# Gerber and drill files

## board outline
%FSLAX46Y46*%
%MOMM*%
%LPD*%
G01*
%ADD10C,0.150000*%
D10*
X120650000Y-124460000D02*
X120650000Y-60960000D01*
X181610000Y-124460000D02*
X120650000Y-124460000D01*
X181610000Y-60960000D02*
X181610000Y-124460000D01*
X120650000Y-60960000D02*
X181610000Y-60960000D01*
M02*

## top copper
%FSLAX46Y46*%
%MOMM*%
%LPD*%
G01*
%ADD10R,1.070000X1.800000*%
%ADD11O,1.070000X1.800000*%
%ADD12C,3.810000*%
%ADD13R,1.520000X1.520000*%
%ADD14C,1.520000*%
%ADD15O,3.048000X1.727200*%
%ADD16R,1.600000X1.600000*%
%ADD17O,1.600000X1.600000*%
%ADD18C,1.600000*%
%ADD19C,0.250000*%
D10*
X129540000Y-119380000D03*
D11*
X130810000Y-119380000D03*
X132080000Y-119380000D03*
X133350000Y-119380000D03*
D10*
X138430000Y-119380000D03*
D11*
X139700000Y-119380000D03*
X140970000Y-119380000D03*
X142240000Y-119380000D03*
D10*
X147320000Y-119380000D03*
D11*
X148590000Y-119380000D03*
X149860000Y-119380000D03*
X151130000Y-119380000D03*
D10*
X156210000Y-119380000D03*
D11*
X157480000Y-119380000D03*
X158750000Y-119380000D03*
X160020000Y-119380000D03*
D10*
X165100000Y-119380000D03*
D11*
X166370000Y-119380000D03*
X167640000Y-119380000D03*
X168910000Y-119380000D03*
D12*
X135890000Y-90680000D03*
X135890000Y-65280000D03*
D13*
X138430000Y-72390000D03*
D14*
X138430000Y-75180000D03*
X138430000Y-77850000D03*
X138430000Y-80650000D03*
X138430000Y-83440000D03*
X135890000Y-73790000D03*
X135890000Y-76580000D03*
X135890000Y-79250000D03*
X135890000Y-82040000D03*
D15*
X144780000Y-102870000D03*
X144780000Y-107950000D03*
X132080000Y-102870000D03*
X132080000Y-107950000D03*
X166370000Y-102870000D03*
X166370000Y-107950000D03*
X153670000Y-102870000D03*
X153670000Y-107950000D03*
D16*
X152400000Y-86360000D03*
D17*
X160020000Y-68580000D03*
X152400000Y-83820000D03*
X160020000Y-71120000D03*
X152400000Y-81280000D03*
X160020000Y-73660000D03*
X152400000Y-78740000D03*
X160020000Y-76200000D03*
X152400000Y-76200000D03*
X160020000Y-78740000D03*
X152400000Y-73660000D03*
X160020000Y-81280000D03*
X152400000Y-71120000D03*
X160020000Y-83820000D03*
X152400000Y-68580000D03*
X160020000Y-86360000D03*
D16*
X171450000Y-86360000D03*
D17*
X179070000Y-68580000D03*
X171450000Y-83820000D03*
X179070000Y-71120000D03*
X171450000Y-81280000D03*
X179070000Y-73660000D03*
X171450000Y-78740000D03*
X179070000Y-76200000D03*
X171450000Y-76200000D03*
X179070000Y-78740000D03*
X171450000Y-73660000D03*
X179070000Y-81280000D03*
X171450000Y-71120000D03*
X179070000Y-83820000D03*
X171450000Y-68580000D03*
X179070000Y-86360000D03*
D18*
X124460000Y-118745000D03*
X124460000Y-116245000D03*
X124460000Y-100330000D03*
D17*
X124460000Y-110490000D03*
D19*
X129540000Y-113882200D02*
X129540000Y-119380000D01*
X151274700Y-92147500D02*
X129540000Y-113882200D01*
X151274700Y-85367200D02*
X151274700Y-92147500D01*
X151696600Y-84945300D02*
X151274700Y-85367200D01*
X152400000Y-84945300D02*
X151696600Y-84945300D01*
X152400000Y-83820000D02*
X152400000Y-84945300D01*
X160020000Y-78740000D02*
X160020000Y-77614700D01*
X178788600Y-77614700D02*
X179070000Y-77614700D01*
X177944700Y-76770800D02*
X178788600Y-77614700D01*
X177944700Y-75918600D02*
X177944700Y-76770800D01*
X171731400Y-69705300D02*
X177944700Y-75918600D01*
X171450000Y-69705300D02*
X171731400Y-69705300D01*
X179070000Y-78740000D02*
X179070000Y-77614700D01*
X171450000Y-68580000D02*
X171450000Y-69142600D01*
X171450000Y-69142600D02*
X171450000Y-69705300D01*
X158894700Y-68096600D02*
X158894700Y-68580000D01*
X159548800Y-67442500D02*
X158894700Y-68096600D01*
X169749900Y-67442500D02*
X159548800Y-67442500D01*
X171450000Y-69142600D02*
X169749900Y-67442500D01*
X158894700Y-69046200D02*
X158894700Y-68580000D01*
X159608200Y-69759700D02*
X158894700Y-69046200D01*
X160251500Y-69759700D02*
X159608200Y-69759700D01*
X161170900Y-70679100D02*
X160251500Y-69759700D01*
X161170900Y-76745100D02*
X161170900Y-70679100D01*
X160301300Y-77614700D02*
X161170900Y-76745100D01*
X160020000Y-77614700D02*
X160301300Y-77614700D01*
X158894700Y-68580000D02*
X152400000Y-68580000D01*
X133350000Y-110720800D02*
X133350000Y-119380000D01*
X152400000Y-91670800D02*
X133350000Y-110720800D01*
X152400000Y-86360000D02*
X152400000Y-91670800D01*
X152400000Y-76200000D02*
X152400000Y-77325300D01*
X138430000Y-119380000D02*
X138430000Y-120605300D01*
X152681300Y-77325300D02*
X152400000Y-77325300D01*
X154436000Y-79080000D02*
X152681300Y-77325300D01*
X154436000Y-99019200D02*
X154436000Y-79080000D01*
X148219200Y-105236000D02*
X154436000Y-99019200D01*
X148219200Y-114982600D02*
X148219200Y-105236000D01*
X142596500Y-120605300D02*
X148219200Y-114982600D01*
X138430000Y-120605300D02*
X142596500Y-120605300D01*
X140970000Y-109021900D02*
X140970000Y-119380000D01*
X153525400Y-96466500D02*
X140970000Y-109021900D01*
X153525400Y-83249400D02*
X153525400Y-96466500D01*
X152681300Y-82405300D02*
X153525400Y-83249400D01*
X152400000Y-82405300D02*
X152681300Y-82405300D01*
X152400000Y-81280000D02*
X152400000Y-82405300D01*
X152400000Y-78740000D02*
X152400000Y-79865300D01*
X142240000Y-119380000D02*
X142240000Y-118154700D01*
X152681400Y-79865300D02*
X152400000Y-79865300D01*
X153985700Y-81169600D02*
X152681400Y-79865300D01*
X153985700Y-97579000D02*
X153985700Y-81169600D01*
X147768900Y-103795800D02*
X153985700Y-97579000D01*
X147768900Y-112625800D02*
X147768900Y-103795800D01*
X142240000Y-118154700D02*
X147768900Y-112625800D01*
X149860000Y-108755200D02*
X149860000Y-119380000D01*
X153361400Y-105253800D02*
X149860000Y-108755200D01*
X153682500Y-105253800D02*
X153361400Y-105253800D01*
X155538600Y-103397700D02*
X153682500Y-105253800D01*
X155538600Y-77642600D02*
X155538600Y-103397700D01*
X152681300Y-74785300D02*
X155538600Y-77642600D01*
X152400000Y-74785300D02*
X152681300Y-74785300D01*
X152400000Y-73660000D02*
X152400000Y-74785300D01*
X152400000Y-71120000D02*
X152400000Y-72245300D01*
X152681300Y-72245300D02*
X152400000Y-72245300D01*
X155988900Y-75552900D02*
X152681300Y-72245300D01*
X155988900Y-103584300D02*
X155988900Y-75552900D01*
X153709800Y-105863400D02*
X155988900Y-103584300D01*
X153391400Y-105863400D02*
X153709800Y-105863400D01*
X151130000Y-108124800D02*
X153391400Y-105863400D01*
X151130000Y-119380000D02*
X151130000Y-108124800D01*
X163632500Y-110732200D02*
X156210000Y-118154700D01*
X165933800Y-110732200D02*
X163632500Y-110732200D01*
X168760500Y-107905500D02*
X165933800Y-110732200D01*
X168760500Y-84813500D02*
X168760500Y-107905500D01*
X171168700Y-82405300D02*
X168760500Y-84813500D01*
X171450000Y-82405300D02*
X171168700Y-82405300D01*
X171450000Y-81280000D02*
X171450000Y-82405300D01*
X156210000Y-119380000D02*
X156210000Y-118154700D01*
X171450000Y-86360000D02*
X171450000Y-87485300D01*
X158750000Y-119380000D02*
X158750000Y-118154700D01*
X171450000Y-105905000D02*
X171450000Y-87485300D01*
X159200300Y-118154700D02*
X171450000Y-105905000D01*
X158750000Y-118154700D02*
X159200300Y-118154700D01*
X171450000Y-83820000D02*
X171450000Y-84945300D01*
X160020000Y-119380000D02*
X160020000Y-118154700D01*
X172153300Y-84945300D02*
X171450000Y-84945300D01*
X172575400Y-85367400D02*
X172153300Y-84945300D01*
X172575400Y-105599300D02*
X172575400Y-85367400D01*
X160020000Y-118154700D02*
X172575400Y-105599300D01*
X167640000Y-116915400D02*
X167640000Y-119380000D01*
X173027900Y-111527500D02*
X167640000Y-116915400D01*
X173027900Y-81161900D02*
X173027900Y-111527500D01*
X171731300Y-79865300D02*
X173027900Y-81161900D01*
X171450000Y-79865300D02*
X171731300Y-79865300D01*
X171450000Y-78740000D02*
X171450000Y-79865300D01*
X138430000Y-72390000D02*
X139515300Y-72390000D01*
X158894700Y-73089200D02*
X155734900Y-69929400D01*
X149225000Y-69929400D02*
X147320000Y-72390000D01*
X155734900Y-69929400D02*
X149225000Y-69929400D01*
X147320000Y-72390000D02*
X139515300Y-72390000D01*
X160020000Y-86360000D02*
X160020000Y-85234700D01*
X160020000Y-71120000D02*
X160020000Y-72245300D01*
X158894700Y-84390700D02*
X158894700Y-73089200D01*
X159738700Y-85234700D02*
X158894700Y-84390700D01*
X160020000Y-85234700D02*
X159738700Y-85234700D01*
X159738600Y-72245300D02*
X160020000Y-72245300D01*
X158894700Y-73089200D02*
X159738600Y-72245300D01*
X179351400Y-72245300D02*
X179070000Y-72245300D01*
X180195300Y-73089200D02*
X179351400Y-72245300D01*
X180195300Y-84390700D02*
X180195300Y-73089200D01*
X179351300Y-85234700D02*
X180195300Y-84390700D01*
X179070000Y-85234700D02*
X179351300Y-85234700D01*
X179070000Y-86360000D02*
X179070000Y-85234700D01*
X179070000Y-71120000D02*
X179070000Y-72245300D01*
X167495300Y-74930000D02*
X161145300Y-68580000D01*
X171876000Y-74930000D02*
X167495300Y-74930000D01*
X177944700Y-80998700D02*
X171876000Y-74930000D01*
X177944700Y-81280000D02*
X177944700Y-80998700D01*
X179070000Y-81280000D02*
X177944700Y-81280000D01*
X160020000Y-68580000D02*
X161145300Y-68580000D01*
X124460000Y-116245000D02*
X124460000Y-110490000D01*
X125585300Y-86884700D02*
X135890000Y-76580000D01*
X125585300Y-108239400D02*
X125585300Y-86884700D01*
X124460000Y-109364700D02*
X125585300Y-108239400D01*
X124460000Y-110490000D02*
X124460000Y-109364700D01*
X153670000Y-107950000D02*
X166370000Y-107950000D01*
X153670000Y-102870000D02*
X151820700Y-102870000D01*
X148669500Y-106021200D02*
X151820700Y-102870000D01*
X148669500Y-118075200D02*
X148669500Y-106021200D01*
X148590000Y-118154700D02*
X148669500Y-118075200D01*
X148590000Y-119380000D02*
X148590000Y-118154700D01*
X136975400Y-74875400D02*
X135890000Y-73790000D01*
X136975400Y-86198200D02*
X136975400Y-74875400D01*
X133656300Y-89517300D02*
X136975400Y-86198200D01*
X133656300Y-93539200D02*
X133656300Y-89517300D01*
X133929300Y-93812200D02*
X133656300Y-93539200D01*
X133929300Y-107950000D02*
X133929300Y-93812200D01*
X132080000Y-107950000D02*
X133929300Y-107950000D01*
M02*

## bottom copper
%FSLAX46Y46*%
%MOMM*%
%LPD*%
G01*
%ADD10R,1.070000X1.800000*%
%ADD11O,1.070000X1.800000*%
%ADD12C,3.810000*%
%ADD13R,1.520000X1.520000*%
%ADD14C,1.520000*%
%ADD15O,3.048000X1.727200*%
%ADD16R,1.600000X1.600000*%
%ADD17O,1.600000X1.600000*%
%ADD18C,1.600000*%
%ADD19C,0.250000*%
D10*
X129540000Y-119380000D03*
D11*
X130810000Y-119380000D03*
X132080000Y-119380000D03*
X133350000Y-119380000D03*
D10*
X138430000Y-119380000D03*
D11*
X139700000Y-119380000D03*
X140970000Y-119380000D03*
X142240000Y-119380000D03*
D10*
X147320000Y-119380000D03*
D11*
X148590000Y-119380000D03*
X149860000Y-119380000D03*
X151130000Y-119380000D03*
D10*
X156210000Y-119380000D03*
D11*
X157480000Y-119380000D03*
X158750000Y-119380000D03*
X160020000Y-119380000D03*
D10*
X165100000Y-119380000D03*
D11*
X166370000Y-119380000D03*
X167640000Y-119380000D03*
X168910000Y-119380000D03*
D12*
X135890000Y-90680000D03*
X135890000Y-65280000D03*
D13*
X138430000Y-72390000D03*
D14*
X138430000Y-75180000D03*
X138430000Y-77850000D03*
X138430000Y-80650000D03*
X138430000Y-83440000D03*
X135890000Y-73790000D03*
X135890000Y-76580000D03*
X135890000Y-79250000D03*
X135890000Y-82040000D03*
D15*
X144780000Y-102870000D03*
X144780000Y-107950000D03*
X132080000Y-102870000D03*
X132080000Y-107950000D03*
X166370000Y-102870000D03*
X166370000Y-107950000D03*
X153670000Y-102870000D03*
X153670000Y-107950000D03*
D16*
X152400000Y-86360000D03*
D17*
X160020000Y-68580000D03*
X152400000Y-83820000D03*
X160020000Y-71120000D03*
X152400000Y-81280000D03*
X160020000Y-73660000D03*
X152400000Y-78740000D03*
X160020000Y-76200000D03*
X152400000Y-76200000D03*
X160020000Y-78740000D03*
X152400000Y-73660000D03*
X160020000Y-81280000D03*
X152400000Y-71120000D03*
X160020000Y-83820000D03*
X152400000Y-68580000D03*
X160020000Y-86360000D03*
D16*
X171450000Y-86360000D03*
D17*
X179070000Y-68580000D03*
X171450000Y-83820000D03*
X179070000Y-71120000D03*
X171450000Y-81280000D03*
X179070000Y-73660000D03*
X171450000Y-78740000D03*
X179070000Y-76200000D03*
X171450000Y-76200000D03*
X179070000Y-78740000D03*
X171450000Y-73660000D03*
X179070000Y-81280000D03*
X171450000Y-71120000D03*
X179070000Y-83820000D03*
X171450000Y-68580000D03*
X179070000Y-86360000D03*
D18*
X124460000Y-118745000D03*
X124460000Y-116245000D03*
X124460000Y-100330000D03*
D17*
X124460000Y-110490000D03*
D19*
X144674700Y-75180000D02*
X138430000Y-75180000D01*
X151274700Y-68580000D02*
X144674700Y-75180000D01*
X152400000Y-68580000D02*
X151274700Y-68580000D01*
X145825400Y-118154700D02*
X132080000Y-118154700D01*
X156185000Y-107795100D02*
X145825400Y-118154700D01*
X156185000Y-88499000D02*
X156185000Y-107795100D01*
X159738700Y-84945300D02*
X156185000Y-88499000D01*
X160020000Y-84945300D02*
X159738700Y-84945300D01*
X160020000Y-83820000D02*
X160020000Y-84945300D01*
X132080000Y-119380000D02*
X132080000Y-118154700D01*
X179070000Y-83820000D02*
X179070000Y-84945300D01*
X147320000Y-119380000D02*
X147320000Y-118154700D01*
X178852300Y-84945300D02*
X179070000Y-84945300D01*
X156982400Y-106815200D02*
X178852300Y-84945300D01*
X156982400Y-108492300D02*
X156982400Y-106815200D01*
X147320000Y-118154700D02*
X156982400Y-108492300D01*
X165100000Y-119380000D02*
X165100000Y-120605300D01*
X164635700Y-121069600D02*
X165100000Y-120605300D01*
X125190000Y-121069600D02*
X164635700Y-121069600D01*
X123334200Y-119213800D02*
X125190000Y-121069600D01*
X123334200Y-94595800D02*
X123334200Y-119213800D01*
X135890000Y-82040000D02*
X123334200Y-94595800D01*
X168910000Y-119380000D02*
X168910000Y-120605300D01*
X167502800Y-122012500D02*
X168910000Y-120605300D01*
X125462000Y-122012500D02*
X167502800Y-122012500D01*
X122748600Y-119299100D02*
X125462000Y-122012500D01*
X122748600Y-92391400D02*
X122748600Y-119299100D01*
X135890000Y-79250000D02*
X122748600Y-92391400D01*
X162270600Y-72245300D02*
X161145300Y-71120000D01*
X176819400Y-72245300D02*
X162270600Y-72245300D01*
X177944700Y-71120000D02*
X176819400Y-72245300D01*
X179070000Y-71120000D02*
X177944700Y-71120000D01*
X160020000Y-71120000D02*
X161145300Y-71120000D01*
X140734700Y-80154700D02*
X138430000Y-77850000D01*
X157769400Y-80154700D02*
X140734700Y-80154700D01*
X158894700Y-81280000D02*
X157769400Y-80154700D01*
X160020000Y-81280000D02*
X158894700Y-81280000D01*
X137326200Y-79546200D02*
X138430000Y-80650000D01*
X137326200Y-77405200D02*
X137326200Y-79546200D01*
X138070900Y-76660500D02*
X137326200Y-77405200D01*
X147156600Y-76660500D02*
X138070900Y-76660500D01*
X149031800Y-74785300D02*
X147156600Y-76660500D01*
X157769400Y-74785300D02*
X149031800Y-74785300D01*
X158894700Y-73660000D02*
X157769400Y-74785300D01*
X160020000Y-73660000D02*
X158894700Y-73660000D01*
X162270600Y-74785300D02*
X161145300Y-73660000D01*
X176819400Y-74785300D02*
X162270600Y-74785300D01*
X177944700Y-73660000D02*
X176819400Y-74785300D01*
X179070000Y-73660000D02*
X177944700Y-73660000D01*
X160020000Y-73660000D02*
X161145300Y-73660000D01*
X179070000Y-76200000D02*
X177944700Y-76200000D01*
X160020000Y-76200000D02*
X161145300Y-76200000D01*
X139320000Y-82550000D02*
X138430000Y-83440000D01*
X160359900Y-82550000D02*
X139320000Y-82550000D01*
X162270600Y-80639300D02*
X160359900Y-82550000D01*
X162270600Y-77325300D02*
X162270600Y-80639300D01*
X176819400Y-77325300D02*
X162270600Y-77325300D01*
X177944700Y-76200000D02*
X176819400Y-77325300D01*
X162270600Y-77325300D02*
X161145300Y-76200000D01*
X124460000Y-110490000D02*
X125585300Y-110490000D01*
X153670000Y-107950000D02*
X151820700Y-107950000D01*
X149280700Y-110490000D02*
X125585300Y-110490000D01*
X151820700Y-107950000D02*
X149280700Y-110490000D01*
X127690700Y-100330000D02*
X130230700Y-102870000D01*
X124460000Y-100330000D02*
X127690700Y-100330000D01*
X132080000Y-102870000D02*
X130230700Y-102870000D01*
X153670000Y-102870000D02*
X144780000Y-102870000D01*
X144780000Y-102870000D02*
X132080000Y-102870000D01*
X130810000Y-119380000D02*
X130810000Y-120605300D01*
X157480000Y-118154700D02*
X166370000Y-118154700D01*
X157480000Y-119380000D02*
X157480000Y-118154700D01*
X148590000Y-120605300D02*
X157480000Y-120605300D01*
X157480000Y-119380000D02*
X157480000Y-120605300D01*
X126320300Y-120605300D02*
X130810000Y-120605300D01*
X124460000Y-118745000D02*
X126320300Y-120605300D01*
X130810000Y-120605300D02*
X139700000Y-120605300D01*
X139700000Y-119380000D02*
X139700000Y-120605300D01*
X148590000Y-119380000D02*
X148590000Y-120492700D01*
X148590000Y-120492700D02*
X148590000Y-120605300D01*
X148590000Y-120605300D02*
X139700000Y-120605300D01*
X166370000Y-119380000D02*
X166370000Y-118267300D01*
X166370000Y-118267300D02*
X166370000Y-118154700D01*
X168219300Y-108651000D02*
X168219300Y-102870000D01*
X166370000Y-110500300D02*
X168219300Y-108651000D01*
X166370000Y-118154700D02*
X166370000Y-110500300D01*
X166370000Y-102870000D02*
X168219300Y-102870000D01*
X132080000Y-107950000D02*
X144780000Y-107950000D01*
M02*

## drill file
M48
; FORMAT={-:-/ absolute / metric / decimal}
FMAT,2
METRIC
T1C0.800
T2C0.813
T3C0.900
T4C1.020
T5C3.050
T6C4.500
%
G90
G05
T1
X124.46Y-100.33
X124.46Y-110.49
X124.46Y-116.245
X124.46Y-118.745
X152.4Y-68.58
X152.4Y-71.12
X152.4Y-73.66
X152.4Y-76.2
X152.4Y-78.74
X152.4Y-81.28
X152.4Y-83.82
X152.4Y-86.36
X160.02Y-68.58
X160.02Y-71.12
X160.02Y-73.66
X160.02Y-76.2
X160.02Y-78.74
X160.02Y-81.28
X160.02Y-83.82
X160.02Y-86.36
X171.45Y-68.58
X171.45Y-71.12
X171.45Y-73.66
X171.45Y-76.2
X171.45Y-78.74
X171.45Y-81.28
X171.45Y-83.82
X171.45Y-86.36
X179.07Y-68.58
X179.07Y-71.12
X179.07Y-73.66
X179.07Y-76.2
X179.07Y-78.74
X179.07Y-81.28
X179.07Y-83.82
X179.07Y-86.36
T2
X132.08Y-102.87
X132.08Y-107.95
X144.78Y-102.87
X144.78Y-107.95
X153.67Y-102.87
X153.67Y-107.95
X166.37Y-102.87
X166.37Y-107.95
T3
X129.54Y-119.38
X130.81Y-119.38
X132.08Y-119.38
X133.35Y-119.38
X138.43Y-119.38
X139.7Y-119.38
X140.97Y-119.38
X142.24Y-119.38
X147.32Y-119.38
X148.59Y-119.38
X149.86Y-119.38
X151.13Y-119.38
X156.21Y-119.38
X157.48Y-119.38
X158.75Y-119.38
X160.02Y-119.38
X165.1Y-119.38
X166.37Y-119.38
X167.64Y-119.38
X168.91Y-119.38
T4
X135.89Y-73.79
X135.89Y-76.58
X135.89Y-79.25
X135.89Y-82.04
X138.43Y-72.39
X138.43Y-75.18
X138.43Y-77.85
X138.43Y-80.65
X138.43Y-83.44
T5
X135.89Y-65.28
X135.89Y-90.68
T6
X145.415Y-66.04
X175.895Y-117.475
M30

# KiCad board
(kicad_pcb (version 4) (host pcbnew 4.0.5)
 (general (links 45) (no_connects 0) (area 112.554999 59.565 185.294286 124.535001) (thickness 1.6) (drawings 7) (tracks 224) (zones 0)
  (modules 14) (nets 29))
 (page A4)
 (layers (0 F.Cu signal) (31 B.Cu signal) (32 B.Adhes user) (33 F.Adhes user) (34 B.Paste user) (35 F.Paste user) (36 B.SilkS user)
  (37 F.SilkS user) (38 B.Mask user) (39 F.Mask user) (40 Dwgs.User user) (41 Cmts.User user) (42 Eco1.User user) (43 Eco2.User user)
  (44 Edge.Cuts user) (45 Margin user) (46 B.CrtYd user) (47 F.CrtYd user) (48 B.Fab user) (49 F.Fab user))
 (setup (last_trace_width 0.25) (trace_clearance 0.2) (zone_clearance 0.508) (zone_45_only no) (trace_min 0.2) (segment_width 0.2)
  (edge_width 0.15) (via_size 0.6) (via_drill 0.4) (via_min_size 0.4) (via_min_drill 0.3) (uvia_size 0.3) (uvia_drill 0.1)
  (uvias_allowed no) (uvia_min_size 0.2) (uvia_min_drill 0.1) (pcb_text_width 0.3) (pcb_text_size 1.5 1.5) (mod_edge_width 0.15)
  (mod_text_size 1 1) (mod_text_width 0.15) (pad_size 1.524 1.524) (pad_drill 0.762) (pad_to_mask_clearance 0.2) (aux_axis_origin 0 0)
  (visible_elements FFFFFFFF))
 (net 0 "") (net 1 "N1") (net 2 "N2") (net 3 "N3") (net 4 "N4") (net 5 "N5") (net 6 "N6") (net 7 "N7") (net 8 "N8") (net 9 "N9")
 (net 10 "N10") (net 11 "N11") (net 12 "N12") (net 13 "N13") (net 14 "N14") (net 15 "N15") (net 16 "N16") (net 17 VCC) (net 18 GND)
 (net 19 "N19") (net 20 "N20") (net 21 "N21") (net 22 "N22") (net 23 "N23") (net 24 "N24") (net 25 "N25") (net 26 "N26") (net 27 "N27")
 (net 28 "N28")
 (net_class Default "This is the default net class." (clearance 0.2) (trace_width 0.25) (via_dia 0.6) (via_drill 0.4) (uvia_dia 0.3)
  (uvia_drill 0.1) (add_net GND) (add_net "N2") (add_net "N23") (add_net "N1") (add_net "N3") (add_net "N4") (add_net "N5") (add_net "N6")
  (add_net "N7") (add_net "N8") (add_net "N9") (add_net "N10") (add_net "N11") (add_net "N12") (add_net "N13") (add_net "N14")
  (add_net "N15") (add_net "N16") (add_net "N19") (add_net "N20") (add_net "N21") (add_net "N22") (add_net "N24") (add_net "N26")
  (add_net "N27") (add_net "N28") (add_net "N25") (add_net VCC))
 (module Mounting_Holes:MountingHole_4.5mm (layer F.Cu) (at 145.415 66.04)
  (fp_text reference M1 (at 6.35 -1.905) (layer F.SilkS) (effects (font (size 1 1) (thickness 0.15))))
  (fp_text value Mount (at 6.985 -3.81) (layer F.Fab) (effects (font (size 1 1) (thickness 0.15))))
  (pad 1 np_thru_hole circle (at 0 0) (size 4.5 4.5) (drill 4.5) (layers *.Cu *.Mask)))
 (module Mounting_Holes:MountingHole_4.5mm (layer F.Cu) (at 175.895 117.475)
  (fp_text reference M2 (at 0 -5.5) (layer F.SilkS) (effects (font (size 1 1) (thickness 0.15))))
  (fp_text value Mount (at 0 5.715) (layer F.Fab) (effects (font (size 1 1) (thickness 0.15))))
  (pad 1 np_thru_hole circle (at 0 0) (size 4.5 4.5) (drill 4.5) (layers *.Cu *.Mask)))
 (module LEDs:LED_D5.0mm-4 (layer F.Cu) (at 129.54 119.38)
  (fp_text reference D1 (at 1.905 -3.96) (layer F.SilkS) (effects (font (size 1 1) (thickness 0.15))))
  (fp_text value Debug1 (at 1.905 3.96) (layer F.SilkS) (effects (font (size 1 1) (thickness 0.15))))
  (pad 1 thru_hole rect (at 0 0) (size 1.07 1.8) (drill 0.9) (layers *.Cu *.Mask) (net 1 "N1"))
  (pad 2 thru_hole oval (at 1.27 0) (size 1.07 1.8) (drill 0.9) (layers *.Cu *.Mask) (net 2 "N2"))
  (pad 3 thru_hole oval (at 2.54 0) (size 1.07 1.8) (drill 0.9) (layers *.Cu *.Mask) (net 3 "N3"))
  (pad 4 thru_hole oval (at 3.81 0) (size 1.07 1.8) (drill 0.9) (layers *.Cu *.Mask) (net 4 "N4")))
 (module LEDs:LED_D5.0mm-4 (layer F.Cu) (at 138.43 119.38)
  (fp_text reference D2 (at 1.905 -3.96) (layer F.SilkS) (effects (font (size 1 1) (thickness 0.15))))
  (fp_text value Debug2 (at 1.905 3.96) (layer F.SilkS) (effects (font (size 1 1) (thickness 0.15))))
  (pad 1 thru_hole rect (at 0 0) (size 1.07 1.8) (drill 0.9) (layers *.Cu *.Mask) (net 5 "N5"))
  (pad 2 thru_hole oval (at 1.27 0) (size 1.07 1.8) (drill 0.9) (layers *.Cu *.Mask) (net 2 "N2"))
  (pad 3 thru_hole oval (at 2.54 0) (size 1.07 1.8) (drill 0.9) (layers *.Cu *.Mask) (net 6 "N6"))
  (pad 4 thru_hole oval (at 3.81 0) (size 1.07 1.8) (drill 0.9) (layers *.Cu *.Mask) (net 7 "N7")))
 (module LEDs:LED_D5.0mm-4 (layer F.Cu) (at 147.32 119.38)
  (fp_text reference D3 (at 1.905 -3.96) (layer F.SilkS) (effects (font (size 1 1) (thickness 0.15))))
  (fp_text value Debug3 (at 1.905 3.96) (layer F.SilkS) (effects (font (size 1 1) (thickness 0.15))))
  (pad 1 thru_hole rect (at 0 0) (size 1.07 1.8) (drill 0.9) (layers *.Cu *.Mask) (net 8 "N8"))
  (pad 2 thru_hole oval (at 1.27 0) (size 1.07 1.8) (drill 0.9) (layers *.Cu *.Mask) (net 2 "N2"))
  (pad 3 thru_hole oval (at 2.54 0) (size 1.07 1.8) (drill 0.9) (layers *.Cu *.Mask) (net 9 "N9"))
  (pad 4 thru_hole oval (at 3.81 0) (size 1.07 1.8) (drill 0.9) (layers *.Cu *.Mask) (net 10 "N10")))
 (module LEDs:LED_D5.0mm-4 (layer F.Cu) (at 156.21 119.38)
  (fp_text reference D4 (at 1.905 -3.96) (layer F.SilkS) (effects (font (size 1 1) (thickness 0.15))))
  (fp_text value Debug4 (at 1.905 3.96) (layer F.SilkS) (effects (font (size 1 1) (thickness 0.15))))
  (pad 1 thru_hole rect (at 0 0) (size 1.07 1.8) (drill 0.9) (layers *.Cu *.Mask) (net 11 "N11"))
  (pad 2 thru_hole oval (at 1.27 0) (size 1.07 1.8) (drill 0.9) (layers *.Cu *.Mask) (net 2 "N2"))
  (pad 3 thru_hole oval (at 2.54 0) (size 1.07 1.8) (drill 0.9) (layers *.Cu *.Mask) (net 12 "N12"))
  (pad 4 thru_hole oval (at 3.81 0) (size 1.07 1.8) (drill 0.9) (layers *.Cu *.Mask) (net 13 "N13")))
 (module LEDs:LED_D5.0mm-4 (layer F.Cu) (at 165.1 119.38)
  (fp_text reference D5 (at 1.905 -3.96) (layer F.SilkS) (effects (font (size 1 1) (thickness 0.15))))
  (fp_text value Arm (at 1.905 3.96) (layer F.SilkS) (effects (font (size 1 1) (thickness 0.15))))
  (pad 1 thru_hole rect (at 0 0) (size 1.07 1.8) (drill 0.9) (layers *.Cu *.Mask) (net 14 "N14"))
  (pad 2 thru_hole oval (at 1.27 0) (size 1.07 1.8) (drill 0.9) (layers *.Cu *.Mask) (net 2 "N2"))
  (pad 3 thru_hole oval (at 2.54 0) (size 1.07 1.8) (drill 0.9) (layers *.Cu *.Mask) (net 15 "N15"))
  (pad 4 thru_hole oval (at 3.81 0) (size 1.07 1.8) (drill 0.9) (layers *.Cu *.Mask) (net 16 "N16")))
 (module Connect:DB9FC (layer B.Cu) (at 138.43 72.39 270)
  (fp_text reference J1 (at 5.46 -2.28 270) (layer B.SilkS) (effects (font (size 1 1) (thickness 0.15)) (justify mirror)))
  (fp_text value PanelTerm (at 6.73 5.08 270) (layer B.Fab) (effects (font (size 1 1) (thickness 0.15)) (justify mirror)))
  (pad "" thru_hole circle (at 18.29 2.54 270) (size 3.81 3.81) (drill 3.05) (layers *.Cu *.Mask))
  (pad "" thru_hole circle (at -7.11 2.54 270) (size 3.81 3.81) (drill 3.05) (layers *.Cu *.Mask))
  (pad 1 thru_hole rect (at 0 0 270) (size 1.52 1.52) (drill 1.02) (layers *.Cu *.Mask) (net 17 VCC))
  (pad 2 thru_hole circle (at 2.79 0 270) (size 1.52 1.52) (drill 1.02) (layers *.Cu *.Mask) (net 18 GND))
  (pad 3 thru_hole circle (at 5.46 0 270) (size 1.52 1.52) (drill 1.02) (layers *.Cu *.Mask) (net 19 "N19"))
  (pad 4 thru_hole circle (at 8.26 0 270) (size 1.52 1.52) (drill 1.02) (layers *.Cu *.Mask) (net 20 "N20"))
  (pad 5 thru_hole circle (at 11.05 0 270) (size 1.52 1.52) (drill 1.02) (layers *.Cu *.Mask) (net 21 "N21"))
  (pad 6 thru_hole circle (at 1.4 2.54 270) (size 1.52 1.52) (drill 1.02) (layers *.Cu *.Mask) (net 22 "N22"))
  (pad 7 thru_hole circle (at 4.19 2.54 270) (size 1.52 1.52) (drill 1.02) (layers *.Cu *.Mask) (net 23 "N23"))
  (pad 8 thru_hole circle (at 6.86 2.54 270) (size 1.52 1.52) (drill 1.02) (layers *.Cu *.Mask) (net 16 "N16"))
  (pad 9 thru_hole circle (at 9.65 2.54 270) (size 1.52 1.52) (drill 1.02) (layers *.Cu *.Mask) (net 14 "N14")))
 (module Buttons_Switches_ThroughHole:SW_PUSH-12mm (layer F.Cu) (at 138.43 105.41)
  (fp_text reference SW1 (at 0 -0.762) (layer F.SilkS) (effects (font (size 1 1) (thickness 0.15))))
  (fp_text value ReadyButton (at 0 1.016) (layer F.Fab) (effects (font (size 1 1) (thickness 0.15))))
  (pad 1 thru_hole oval (at 6.35 -2.54) (size 3.048 1.7272) (drill 0.8128) (layers *.Cu *.Mask) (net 2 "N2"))
  (pad 2 thru_hole oval (at 6.35 2.54) (size 3.048 1.7272) (drill 0.8128) (layers *.Cu *.Mask) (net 22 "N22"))
  (pad 1 thru_hole oval (at -6.35 -2.54) (size 3.048 1.7272) (drill 0.8128) (layers *.Cu *.Mask) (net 2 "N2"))
  (pad 2 thru_hole oval (at -6.35 2.54) (size 3.048 1.7272) (drill 0.8128) (layers *.Cu *.Mask) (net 22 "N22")))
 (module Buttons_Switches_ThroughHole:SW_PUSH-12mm (layer F.Cu) (at 160.02 105.41)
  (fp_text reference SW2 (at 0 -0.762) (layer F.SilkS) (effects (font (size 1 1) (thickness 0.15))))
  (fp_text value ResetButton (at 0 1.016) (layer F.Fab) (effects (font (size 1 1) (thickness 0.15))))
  (pad 1 thru_hole oval (at 6.35 -2.54) (size 3.048 1.7272) (drill 0.8128) (layers *.Cu *.Mask) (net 2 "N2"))
  (pad 2 thru_hole oval (at 6.35 2.54) (size 3.048 1.7272) (drill 0.8128) (layers *.Cu *.Mask) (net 23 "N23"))
  (pad 1 thru_hole oval (at -6.35 -2.54) (size 3.048 1.7272) (drill 0.8128) (layers *.Cu *.Mask) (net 2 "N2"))
  (pad 2 thru_hole oval (at -6.35 2.54) (size 3.048 1.7272) (drill 0.8128) (layers *.Cu *.Mask) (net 23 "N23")))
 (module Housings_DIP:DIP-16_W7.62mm (layer B.Cu) (at 152.4 86.36)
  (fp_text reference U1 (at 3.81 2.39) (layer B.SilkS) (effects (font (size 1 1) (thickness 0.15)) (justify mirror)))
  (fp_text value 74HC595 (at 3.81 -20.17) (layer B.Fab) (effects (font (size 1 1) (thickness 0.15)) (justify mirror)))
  (pad 1 thru_hole rect (at 0 0) (size 1.6 1.6) (drill 0.8) (layers *.Cu *.Mask) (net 4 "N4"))
  (pad 9 thru_hole oval (at 7.62 -17.78) (size 1.6 1.6) (drill 0.8) (layers *.Cu *.Mask) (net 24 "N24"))
  (pad 2 thru_hole oval (at 0 -2.54) (size 1.6 1.6) (drill 0.8) (layers *.Cu *.Mask) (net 1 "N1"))
  (pad 10 thru_hole oval (at 7.62 -15.24) (size 1.6 1.6) (drill 0.8) (layers *.Cu *.Mask) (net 17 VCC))
  (pad 3 thru_hole oval (at 0 -5.08) (size 1.6 1.6) (drill 0.8) (layers *.Cu *.Mask) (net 6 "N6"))
  (pad 11 thru_hole oval (at 7.62 -12.7) (size 1.6 1.6) (drill 0.8) (layers *.Cu *.Mask) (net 20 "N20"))
  (pad 4 thru_hole oval (at 0 -7.62) (size 1.6 1.6) (drill 0.8) (layers *.Cu *.Mask) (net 7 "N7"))
  (pad 12 thru_hole oval (at 7.62 -10.16) (size 1.6 1.6) (drill 0.8) (layers *.Cu *.Mask) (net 21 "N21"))
  (pad 5 thru_hole oval (at 0 -10.16) (size 1.6 1.6) (drill 0.8) (layers *.Cu *.Mask) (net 5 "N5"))
  (pad 13 thru_hole oval (at 7.62 -7.62) (size 1.6 1.6) (drill 0.8) (layers *.Cu *.Mask) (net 18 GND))
  (pad 6 thru_hole oval (at 0 -12.7) (size 1.6 1.6) (drill 0.8) (layers *.Cu *.Mask) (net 9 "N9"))
  (pad 14 thru_hole oval (at 7.62 -5.08) (size 1.6 1.6) (drill 0.8) (layers *.Cu *.Mask) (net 19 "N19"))
  (pad 7 thru_hole oval (at 0 -15.24) (size 1.6 1.6) (drill 0.8) (layers *.Cu *.Mask) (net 10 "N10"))
  (pad 15 thru_hole oval (at 7.62 -2.54) (size 1.6 1.6) (drill 0.8) (layers *.Cu *.Mask) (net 3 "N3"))
  (pad 8 thru_hole oval (at 0 -17.78) (size 1.6 1.6) (drill 0.8) (layers *.Cu *.Mask) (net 18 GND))
  (pad 16 thru_hole oval (at 7.62 0) (size 1.6 1.6) (drill 0.8) (layers *.Cu *.Mask) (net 17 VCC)))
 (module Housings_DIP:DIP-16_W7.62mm (layer B.Cu) (at 171.45 86.36)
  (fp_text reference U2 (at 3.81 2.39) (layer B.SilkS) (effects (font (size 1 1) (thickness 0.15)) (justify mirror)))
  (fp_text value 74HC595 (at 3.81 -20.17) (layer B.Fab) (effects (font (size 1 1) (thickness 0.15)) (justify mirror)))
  (pad 1 thru_hole rect (at 0 0) (size 1.6 1.6) (drill 0.8) (layers *.Cu *.Mask) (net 12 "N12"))
  (pad 9 thru_hole oval (at 7.62 -17.78) (size 1.6 1.6) (drill 0.8) (layers *.Cu *.Mask) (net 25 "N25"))
  (pad 2 thru_hole oval (at 0 -2.54) (size 1.6 1.6) (drill 0.8) (layers *.Cu *.Mask) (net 13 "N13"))
  (pad 10 thru_hole oval (at 7.62 -15.24) (size 1.6 1.6) (drill 0.8) (layers *.Cu *.Mask) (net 17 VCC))
  (pad 3 thru_hole oval (at 0 -5.08) (size 1.6 1.6) (drill 0.8) (layers *.Cu *.Mask) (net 11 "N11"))
  (pad 11 thru_hole oval (at 7.62 -12.7) (size 1.6 1.6) (drill 0.8) (layers *.Cu *.Mask) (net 20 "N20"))
  (pad 4 thru_hole oval (at 0 -7.62) (size 1.6 1.6) (drill 0.8) (layers *.Cu *.Mask) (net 15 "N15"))
  (pad 12 thru_hole oval (at 7.62 -10.16) (size 1.6 1.6) (drill 0.8) (layers *.Cu *.Mask) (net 21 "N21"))
  (pad 5 thru_hole oval (at 0 -10.16) (size 1.6 1.6) (drill 0.8) (layers *.Cu *.Mask) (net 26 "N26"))
  (pad 13 thru_hole oval (at 7.62 -7.62) (size 1.6 1.6) (drill 0.8) (layers *.Cu *.Mask) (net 18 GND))
  (pad 6 thru_hole oval (at 0 -12.7) (size 1.6 1.6) (drill 0.8) (layers *.Cu *.Mask) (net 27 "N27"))
  (pad 14 thru_hole oval (at 7.62 -5.08) (size 1.6 1.6) (drill 0.8) (layers *.Cu *.Mask) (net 24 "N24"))
  (pad 7 thru_hole oval (at 0 -15.24) (size 1.6 1.6) (drill 0.8) (layers *.Cu *.Mask) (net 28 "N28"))
  (pad 15 thru_hole oval (at 7.62 -2.54) (size 1.6 1.6) (drill 0.8) (layers *.Cu *.Mask) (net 8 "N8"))
  (pad 8 thru_hole oval (at 0 -17.78) (size 1.6 1.6) (drill 0.8) (layers *.Cu *.Mask) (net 18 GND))
  (pad 16 thru_hole oval (at 7.62 0) (size 1.6 1.6) (drill 0.8) (layers *.Cu *.Mask) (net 17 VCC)))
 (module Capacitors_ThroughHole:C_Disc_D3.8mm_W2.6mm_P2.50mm (layer F.Cu) (at 124.46 118.745 90)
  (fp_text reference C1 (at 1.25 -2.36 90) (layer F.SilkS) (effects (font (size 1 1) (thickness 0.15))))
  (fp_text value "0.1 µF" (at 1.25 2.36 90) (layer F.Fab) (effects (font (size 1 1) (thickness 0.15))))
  (pad 1 thru_hole circle (at 0 0 90) (size 1.6 1.6) (drill 0.8) (layers *.Cu *.Mask) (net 2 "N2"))
  (pad 2 thru_hole circle (at 2.5 0 90) (size 1.6 1.6) (drill 0.8) (layers *.Cu *.Mask) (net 23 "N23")))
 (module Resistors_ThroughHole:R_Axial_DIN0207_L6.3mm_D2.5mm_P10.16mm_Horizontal (layer F.Cu) (at 124.46 100.33 270)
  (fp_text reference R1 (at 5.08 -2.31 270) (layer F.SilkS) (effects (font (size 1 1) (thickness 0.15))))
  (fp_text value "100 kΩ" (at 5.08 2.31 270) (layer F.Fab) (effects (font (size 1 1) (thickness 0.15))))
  (pad 1 thru_hole circle (at 0 0 270) (size 1.6 1.6) (drill 0.8) (layers *.Cu *.Mask) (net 2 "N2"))
  (pad 2 thru_hole oval (at 10.16 0 270) (size 1.6 1.6) (drill 0.8) (layers *.Cu *.Mask) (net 23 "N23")))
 (gr_line (start 120.65 124.46) (end 120.65 60.96) (angle 90) (layer Edge.Cuts) (width 0.15))
 (gr_line (start 181.61 124.46) (end 120.65 124.46) (angle 90) (layer Edge.Cuts) (width 0.15))
 (gr_line (start 181.61 60.96) (end 181.61 124.46) (angle 90) (layer Edge.Cuts) (width 0.15))
 (gr_line (start 120.65 60.96) (end 181.61 60.96) (angle 90) (layer Edge.Cuts) (width 0.15))
 (segment (start 129.54 113.8822) (end 129.54 119.38) (width 0.25) (layer F.Cu) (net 1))
 (segment (start 151.2747 92.1475) (end 129.54 113.8822) (width 0.25) (layer F.Cu) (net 1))
 (segment (start 151.2747 85.3672) (end 151.2747 92.1475) (width 0.25) (layer F.Cu) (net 1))
 (segment (start 151.6966 84.9453) (end 151.2747 85.3672) (width 0.25) (layer F.Cu) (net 1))
 (segment (start 152.4 84.9453) (end 151.6966 84.9453) (width 0.25) (layer F.Cu) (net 1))
 (segment (start 152.4 83.82) (end 152.4 84.9453) (width 0.25) (layer F.Cu) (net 1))
 (segment (start 144.6747 75.18) (end 138.43 75.18) (width 0.25) (layer B.Cu) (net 18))
 (segment (start 151.2747 68.58) (end 144.6747 75.18) (width 0.25) (layer B.Cu) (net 18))
 (segment (start 152.4 68.58) (end 151.2747 68.58) (width 0.25) (layer B.Cu) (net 18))
 (segment (start 160.02 78.74) (end 160.02 77.6147) (width 0.25) (layer F.Cu) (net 18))
 (segment (start 178.7886 77.6147) (end 179.07 77.6147) (width 0.25) (layer F.Cu) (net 18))
 (segment (start 177.9447 76.7708) (end 178.7886 77.6147) (width 0.25) (layer F.Cu) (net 18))
 (segment (start 177.9447 75.9186) (end 177.9447 76.7708) (width 0.25) (layer F.Cu) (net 18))
 (segment (start 171.7314 69.7053) (end 177.9447 75.9186) (width 0.25) (layer F.Cu) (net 18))
 (segment (start 171.45 69.7053) (end 171.7314 69.7053) (width 0.25) (layer F.Cu) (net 18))
 (segment (start 179.07 78.74) (end 179.07 77.6147) (width 0.25) (layer F.Cu) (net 18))
 (segment (start 171.45 68.58) (end 171.45 69.1426) (width 0.25) (layer F.Cu) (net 18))
 (segment (start 171.45 69.1426) (end 171.45 69.7053) (width 0.25) (layer F.Cu) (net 18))
 (segment (start 158.8947 68.0966) (end 158.8947 68.58) (width 0.25) (layer F.Cu) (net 18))
 (segment (start 159.5488 67.4425) (end 158.8947 68.0966) (width 0.25) (layer F.Cu) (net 18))
 (segment (start 169.7499 67.4425) (end 159.5488 67.4425) (width 0.25) (layer F.Cu) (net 18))
 (segment (start 171.45 69.1426) (end 169.7499 67.4425) (width 0.25) (layer F.Cu) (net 18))
 (segment (start 158.8947 69.0462) (end 158.8947 68.58) (width 0.25) (layer F.Cu) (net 18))
 (segment (start 159.6082 69.7597) (end 158.8947 69.0462) (width 0.25) (layer F.Cu) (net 18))
 (segment (start 160.2515 69.7597) (end 159.6082 69.7597) (width 0.25) (layer F.Cu) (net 18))
 (segment (start 161.1709 70.6791) (end 160.2515 69.7597) (width 0.25) (layer F.Cu) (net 18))
 (segment (start 161.1709 76.7451) (end 161.1709 70.6791) (width 0.25) (layer F.Cu) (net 18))
 (segment (start 160.3013 77.6147) (end 161.1709 76.7451) (width 0.25) (layer F.Cu) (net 18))
 (segment (start 160.02 77.6147) (end 160.3013 77.6147) (width 0.25) (layer F.Cu) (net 18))
 (segment (start 158.8947 68.58) (end 152.4 68.58) (width 0.25) (layer F.Cu) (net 18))
 (segment (start 145.8254 118.1547) (end 132.08 118.1547) (width 0.25) (layer B.Cu) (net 3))
 (segment (start 156.185 107.7951) (end 145.8254 118.1547) (width 0.25) (layer B.Cu) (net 3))
 (segment (start 156.185 88.499) (end 156.185 107.7951) (width 0.25) (layer B.Cu) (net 3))
 (segment (start 159.7387 84.9453) (end 156.185 88.499) (width 0.25) (layer B.Cu) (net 3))
 (segment (start 160.02 84.9453) (end 159.7387 84.9453) (width 0.25) (layer B.Cu) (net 3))
 (segment (start 160.02 83.82) (end 160.02 84.9453) (width 0.25) (layer B.Cu) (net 3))
 (segment (start 132.08 119.38) (end 132.08 118.1547) (width 0.25) (layer B.Cu) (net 3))
 (segment (start 133.35 110.7208) (end 133.35 119.38) (width 0.25) (layer F.Cu) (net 4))
 (segment (start 152.4 91.6708) (end 133.35 110.7208) (width 0.25) (layer F.Cu) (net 4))
 (segment (start 152.4 86.36) (end 152.4 91.6708) (width 0.25) (layer F.Cu) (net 4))
 (segment (start 152.4 76.2) (end 152.4 77.3253) (width 0.25) (layer F.Cu) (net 5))
 (segment (start 138.43 119.38) (end 138.43 120.6053) (width 0.25) (layer F.Cu) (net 5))
 (segment (start 152.6813 77.3253) (end 152.4 77.3253) (width 0.25) (layer F.Cu) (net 5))
 (segment (start 154.436 79.08) (end 152.6813 77.3253) (width 0.25) (layer F.Cu) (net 5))
 (segment (start 154.436 99.0192) (end 154.436 79.08) (width 0.25) (layer F.Cu) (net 5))
 (segment (start 148.2192 105.236) (end 154.436 99.0192) (width 0.25) (layer F.Cu) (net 5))
 (segment (start 148.2192 114.9826) (end 148.2192 105.236) (width 0.25) (layer F.Cu) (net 5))
 (segment (start 142.5965 120.6053) (end 148.2192 114.9826) (width 0.25) (layer F.Cu) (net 5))
 (segment (start 138.43 120.6053) (end 142.5965 120.6053) (width 0.25) (layer F.Cu) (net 5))
 (segment (start 140.97 109.0219) (end 140.97 119.38) (width 0.25) (layer F.Cu) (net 6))
 (segment (start 153.5254 96.4665) (end 140.97 109.0219) (width 0.25) (layer F.Cu) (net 6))
 (segment (start 153.5254 83.2494) (end 153.5254 96.4665) (width 0.25) (layer F.Cu) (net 6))
 (segment (start 152.6813 82.4053) (end 153.5254 83.2494) (width 0.25) (layer F.Cu) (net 6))
 (segment (start 152.4 82.4053) (end 152.6813 82.4053) (width 0.25) (layer F.Cu) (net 6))
 (segment (start 152.4 81.28) (end 152.4 82.4053) (width 0.25) (layer F.Cu) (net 6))
 (segment (start 152.4 78.74) (end 152.4 79.8653) (width 0.25) (layer F.Cu) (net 7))
 (segment (start 142.24 119.38) (end 142.24 118.1547) (width 0.25) (layer F.Cu) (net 7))
 (segment (start 152.6814 79.8653) (end 152.4 79.8653) (width 0.25) (layer F.Cu) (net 7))
 (segment (start 153.9857 81.1696) (end 152.6814 79.8653) (width 0.25) (layer F.Cu) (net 7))
 (segment (start 153.9857 97.579) (end 153.9857 81.1696) (width 0.25) (layer F.Cu) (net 7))
 (segment (start 147.7689 103.7958) (end 153.9857 97.579) (width 0.25) (layer F.Cu) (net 7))
 (segment (start 147.7689 112.6258) (end 147.7689 103.7958) (width 0.25) (layer F.Cu) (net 7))
 (segment (start 142.24 118.1547) (end 147.7689 112.6258) (width 0.25) (layer F.Cu) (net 7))
 (segment (start 179.07 83.82) (end 179.07 84.9453) (width 0.25) (layer B.Cu) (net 8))
 (segment (start 147.32 119.38) (end 147.32 118.1547) (width 0.25) (layer B.Cu) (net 8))
 (segment (start 178.8523 84.9453) (end 179.07 84.9453) (width 0.25) (layer B.Cu) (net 8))
 (segment (start 156.9824 106.8152) (end 178.8523 84.9453) (width 0.25) (layer B.Cu) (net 8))
 (segment (start 156.9824 108.4923) (end 156.9824 106.8152) (width 0.25) (layer B.Cu) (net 8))
 (segment (start 147.32 118.1547) (end 156.9824 108.4923) (width 0.25) (layer B.Cu) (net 8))
 (segment (start 149.86 108.7552) (end 149.86 119.38) (width 0.25) (layer F.Cu) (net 9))
 (segment (start 153.3614 105.2538) (end 149.86 108.7552) (width 0.25) (layer F.Cu) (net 9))
 (segment (start 153.6825 105.2538) (end 153.3614 105.2538) (width 0.25) (layer F.Cu) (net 9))
 (segment (start 155.5386 103.3977) (end 153.6825 105.2538) (width 0.25) (layer F.Cu) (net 9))
 (segment (start 155.5386 77.6426) (end 155.5386 103.3977) (width 0.25) (layer F.Cu) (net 9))
 (segment (start 152.6813 74.7853) (end 155.5386 77.6426) (width 0.25) (layer F.Cu) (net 9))
 (segment (start 152.4 74.7853) (end 152.6813 74.7853) (width 0.25) (layer F.Cu) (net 9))
 (segment (start 152.4 73.66) (end 152.4 74.7853) (width 0.25) (layer F.Cu) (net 9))
 (segment (start 152.4 71.12) (end 152.4 72.2453) (width 0.25) (layer F.Cu) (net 10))
 (segment (start 152.6813 72.2453) (end 152.4 72.2453) (width 0.25) (layer F.Cu) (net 10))
 (segment (start 155.9889 75.5529) (end 152.6813 72.2453) (width 0.25) (layer F.Cu) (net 10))
 (segment (start 155.9889 103.5843) (end 155.9889 75.5529) (width 0.25) (layer F.Cu) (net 10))
 (segment (start 153.7098 105.8634) (end 155.9889 103.5843) (width 0.25) (layer F.Cu) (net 10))
 (segment (start 153.3914 105.8634) (end 153.7098 105.8634) (width 0.25) (layer F.Cu) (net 10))
 (segment (start 151.13 108.1248) (end 153.3914 105.8634) (width 0.25) (layer F.Cu) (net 10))
 (segment (start 151.13 119.38) (end 151.13 108.1248) (width 0.25) (layer F.Cu) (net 10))
 (segment (start 163.6325 110.7322) (end 156.21 118.1547) (width 0.25) (layer F.Cu) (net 11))
 (segment (start 165.9338 110.7322) (end 163.6325 110.7322) (width 0.25) (layer F.Cu) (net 11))
 (segment (start 168.7605 107.9055) (end 165.9338 110.7322) (width 0.25) (layer F.Cu) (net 11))
 (segment (start 168.7605 84.8135) (end 168.7605 107.9055) (width 0.25) (layer F.Cu) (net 11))
 (segment (start 171.1687 82.4053) (end 168.7605 84.8135) (width 0.25) (layer F.Cu) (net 11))
 (segment (start 171.45 82.4053) (end 171.1687 82.4053) (width 0.25) (layer F.Cu) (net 11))
 (segment (start 171.45 81.28) (end 171.45 82.4053) (width 0.25) (layer F.Cu) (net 11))
 (segment (start 156.21 119.38) (end 156.21 118.1547) (width 0.25) (layer F.Cu) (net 11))
 (segment (start 171.45 86.36) (end 171.45 87.4853) (width 0.25) (layer F.Cu) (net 12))
 (segment (start 158.75 119.38) (end 158.75 118.1547) (width 0.25) (layer F.Cu) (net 12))
 (segment (start 171.45 105.905) (end 171.45 87.4853) (width 0.25) (layer F.Cu) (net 12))
 (segment (start 159.2003 118.1547) (end 171.45 105.905) (width 0.25) (layer F.Cu) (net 12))
 (segment (start 158.75 118.1547) (end 159.2003 118.1547) (width 0.25) (layer F.Cu) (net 12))
 (segment (start 171.45 83.82) (end 171.45 84.9453) (width 0.25) (layer F.Cu) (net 13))
 (segment (start 160.02 119.38) (end 160.02 118.1547) (width 0.25) (layer F.Cu) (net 13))
 (segment (start 172.1533 84.9453) (end 171.45 84.9453) (width 0.25) (layer F.Cu) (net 13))
 (segment (start 172.5754 85.3674) (end 172.1533 84.9453) (width 0.25) (layer F.Cu) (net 13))
 (segment (start 172.5754 105.5993) (end 172.5754 85.3674) (width 0.25) (layer F.Cu) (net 13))
 (segment (start 160.02 118.1547) (end 172.5754 105.5993) (width 0.25) (layer F.Cu) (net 13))
 (segment (start 165.1 119.38) (end 165.1 120.6053) (width 0.25) (layer B.Cu) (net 14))
 (segment (start 164.6357 121.0696) (end 165.1 120.6053) (width 0.25) (layer B.Cu) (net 14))
 (segment (start 125.19 121.0696) (end 164.6357 121.0696) (width 0.25) (layer B.Cu) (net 14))
 (segment (start 123.3342 119.2138) (end 125.19 121.0696) (width 0.25) (layer B.Cu) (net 14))
 (segment (start 123.3342 94.5958) (end 123.3342 119.2138) (width 0.25) (layer B.Cu) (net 14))
 (segment (start 135.89 82.04) (end 123.3342 94.5958) (width 0.25) (layer B.Cu) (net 14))
 (segment (start 167.64 116.9154) (end 167.64 119.38) (width 0.25) (layer F.Cu) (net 15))
 (segment (start 173.0279 111.5275) (end 167.64 116.9154) (width 0.25) (layer F.Cu) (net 15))
 (segment (start 173.0279 81.1619) (end 173.0279 111.5275) (width 0.25) (layer F.Cu) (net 15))
 (segment (start 171.7313 79.8653) (end 173.0279 81.1619) (width 0.25) (layer F.Cu) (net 15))
 (segment (start 171.45 79.8653) (end 171.7313 79.8653) (width 0.25) (layer F.Cu) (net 15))
 (segment (start 171.45 78.74) (end 171.45 79.8653) (width 0.25) (layer F.Cu) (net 15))
 (segment (start 168.91 119.38) (end 168.91 120.6053) (width 0.25) (layer B.Cu) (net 16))
 (segment (start 167.5028 122.0125) (end 168.91 120.6053) (width 0.25) (layer B.Cu) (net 16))
 (segment (start 125.462 122.0125) (end 167.5028 122.0125) (width 0.25) (layer B.Cu) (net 16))
 (segment (start 122.7486 119.2991) (end 125.462 122.0125) (width 0.25) (layer B.Cu) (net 16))
 (segment (start 122.7486 92.3914) (end 122.7486 119.2991) (width 0.25) (layer B.Cu) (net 16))
 (segment (start 135.89 79.25) (end 122.7486 92.3914) (width 0.25) (layer B.Cu) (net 16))
 (segment (start 138.43 72.39) (end 139.5153 72.39) (width 0.25) (layer F.Cu) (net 17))
 (segment (start 158.8947 73.0892) (end 155.7349 69.9294) (width 0.25) (layer F.Cu) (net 17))
 (segment (start 149.225 69.9294) (end 147.32 72.39) (width 0.25) (layer F.Cu) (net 17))
 (segment (start 155.7349 69.9294) (end 149.225 69.9294) (width 0.25) (layer F.Cu) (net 17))
 (segment (start 147.32 72.39) (end 139.5153 72.39) (width 0.25) (layer F.Cu) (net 17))
 (segment (start 160.02 86.36) (end 160.02 85.2347) (width 0.25) (layer F.Cu) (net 17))
 (segment (start 160.02 71.12) (end 160.02 72.2453) (width 0.25) (layer F.Cu) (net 17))
 (segment (start 158.8947 84.3907) (end 158.8947 73.0892) (width 0.25) (layer F.Cu) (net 17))
 (segment (start 159.7387 85.2347) (end 158.8947 84.3907) (width 0.25) (layer F.Cu) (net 17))
 (segment (start 160.02 85.2347) (end 159.7387 85.2347) (width 0.25) (layer F.Cu) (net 17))
 (segment (start 159.7386 72.2453) (end 160.02 72.2453) (width 0.25) (layer F.Cu) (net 17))
 (segment (start 158.8947 73.0892) (end 159.7386 72.2453) (width 0.25) (layer F.Cu) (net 17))
 (segment (start 179.3514 72.2453) (end 179.07 72.2453) (width 0.25) (layer F.Cu) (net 17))
 (segment (start 180.1953 73.0892) (end 179.3514 72.2453) (width 0.25) (layer F.Cu) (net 17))
 (segment (start 180.1953 84.3907) (end 180.1953 73.0892) (width 0.25) (layer F.Cu) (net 17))
 (segment (start 179.3513 85.2347) (end 180.1953 84.3907) (width 0.25) (layer F.Cu) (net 17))
 (segment (start 179.07 85.2347) (end 179.3513 85.2347) (width 0.25) (layer F.Cu) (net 17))
 (segment (start 179.07 86.36) (end 179.07 85.2347) (width 0.25) (layer F.Cu) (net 17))
 (segment (start 179.07 71.12) (end 179.07 72.2453) (width 0.25) (layer F.Cu) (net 17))
 (segment (start 162.2706 72.2453) (end 161.1453 71.12) (width 0.25) (layer B.Cu) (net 17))
 (segment (start 176.8194 72.2453) (end 162.2706 72.2453) (width 0.25) (layer B.Cu) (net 17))
 (segment (start 177.9447 71.12) (end 176.8194 72.2453) (width 0.25) (layer B.Cu) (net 17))
 (segment (start 179.07 71.12) (end 177.9447 71.12) (width 0.25) (layer B.Cu) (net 17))
 (segment (start 160.02 71.12) (end 161.1453 71.12) (width 0.25) (layer B.Cu) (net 17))
 (segment (start 140.7347 80.1547) (end 138.43 77.85) (width 0.25) (layer B.Cu) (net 19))
 (segment (start 157.7694 80.1547) (end 140.7347 80.1547) (width 0.25) (layer B.Cu) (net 19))
 (segment (start 158.8947 81.28) (end 157.7694 80.1547) (width 0.25) (layer B.Cu) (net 19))
 (segment (start 160.02 81.28) (end 158.8947 81.28) (width 0.25) (layer B.Cu) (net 19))
 (segment (start 137.3262 79.5462) (end 138.43 80.65) (width 0.25) (layer B.Cu) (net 20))
 (segment (start 137.3262 77.4052) (end 137.3262 79.5462) (width 0.25) (layer B.Cu) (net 20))
 (segment (start 138.0709 76.6605) (end 137.3262 77.4052) (width 0.25) (layer B.Cu) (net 20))
 (segment (start 147.1566 76.6605) (end 138.0709 76.6605) (width 0.25) (layer B.Cu) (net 20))
 (segment (start 149.0318 74.7853) (end 147.1566 76.6605) (width 0.25) (layer B.Cu) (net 20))
 (segment (start 157.7694 74.7853) (end 149.0318 74.7853) (width 0.25) (layer B.Cu) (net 20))
 (segment (start 158.8947 73.66) (end 157.7694 74.7853) (width 0.25) (layer B.Cu) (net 20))
 (segment (start 160.02 73.66) (end 158.8947 73.66) (width 0.25) (layer B.Cu) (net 20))
 (segment (start 162.2706 74.7853) (end 161.1453 73.66) (width 0.25) (layer B.Cu) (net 20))
 (segment (start 176.8194 74.7853) (end 162.2706 74.7853) (width 0.25) (layer B.Cu) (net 20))
 (segment (start 177.9447 73.66) (end 176.8194 74.7853) (width 0.25) (layer B.Cu) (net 20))
 (segment (start 179.07 73.66) (end 177.9447 73.66) (width 0.25) (layer B.Cu) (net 20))
 (segment (start 160.02 73.66) (end 161.1453 73.66) (width 0.25) (layer B.Cu) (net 20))
 (segment (start 179.07 76.2) (end 177.9447 76.2) (width 0.25) (layer B.Cu) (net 21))
 (segment (start 160.02 76.2) (end 161.1453 76.2) (width 0.25) (layer B.Cu) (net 21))
 (segment (start 139.32 82.55) (end 138.43 83.44) (width 0.25) (layer B.Cu) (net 21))
 (segment (start 160.3599 82.55) (end 139.32 82.55) (width 0.25) (layer B.Cu) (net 21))
 (segment (start 162.2706 80.6393) (end 160.3599 82.55) (width 0.25) (layer B.Cu) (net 21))
 (segment (start 162.2706 77.3253) (end 162.2706 80.6393) (width 0.25) (layer B.Cu) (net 21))
 (segment (start 176.8194 77.3253) (end 162.2706 77.3253) (width 0.25) (layer B.Cu) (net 21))
 (segment (start 177.9447 76.2) (end 176.8194 77.3253) (width 0.25) (layer B.Cu) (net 21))
 (segment (start 162.2706 77.3253) (end 161.1453 76.2) (width 0.25) (layer B.Cu) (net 21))
 (segment (start 167.4953 74.93) (end 161.1453 68.58) (width 0.25) (layer F.Cu) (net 24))
 (segment (start 171.876 74.93) (end 167.4953 74.93) (width 0.25) (layer F.Cu) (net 24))
 (segment (start 177.9447 80.9987) (end 171.876 74.93) (width 0.25) (layer F.Cu) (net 24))
 (segment (start 177.9447 81.28) (end 177.9447 80.9987) (width 0.25) (layer F.Cu) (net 24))
 (segment (start 179.07 81.28) (end 177.9447 81.28) (width 0.25) (layer F.Cu) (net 24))
 (segment (start 160.02 68.58) (end 161.1453 68.58) (width 0.25) (layer F.Cu) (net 24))
 (segment (start 124.46 116.245) (end 124.46 110.49) (width 0.25) (layer F.Cu) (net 23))
 (segment (start 125.5853 86.8847) (end 135.89 76.58) (width 0.25) (layer F.Cu) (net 23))
 (segment (start 125.5853 108.2394) (end 125.5853 86.8847) (width 0.25) (layer F.Cu) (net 23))
 (segment (start 124.46 109.3647) (end 125.5853 108.2394) (width 0.25) (layer F.Cu) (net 23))
 (segment (start 124.46 110.49) (end 124.46 109.3647) (width 0.25) (layer F.Cu) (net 23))
 (segment (start 124.46 110.49) (end 125.5853 110.49) (width 0.25) (layer B.Cu) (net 23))
 (segment (start 153.67 107.95) (end 151.8207 107.95) (width 0.25) (layer B.Cu) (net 23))
 (segment (start 149.2807 110.49) (end 125.5853 110.49) (width 0.25) (layer B.Cu) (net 23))
 (segment (start 151.8207 107.95) (end 149.2807 110.49) (width 0.25) (layer B.Cu) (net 23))
 (segment (start 153.67 107.95) (end 166.37 107.95) (width 0.25) (layer F.Cu) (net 23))
 (segment (start 127.6907 100.33) (end 130.2307 102.87) (width 0.25) (layer B.Cu) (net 2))
 (segment (start 124.46 100.33) (end 127.6907 100.33) (width 0.25) (layer B.Cu) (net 2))
 (segment (start 132.08 102.87) (end 130.2307 102.87) (width 0.25) (layer B.Cu) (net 2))
 (segment (start 153.67 102.87) (end 144.78 102.87) (width 0.25) (layer B.Cu) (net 2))
 (segment (start 144.78 102.87) (end 132.08 102.87) (width 0.25) (layer B.Cu) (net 2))
 (segment (start 153.67 102.87) (end 151.8207 102.87) (width 0.25) (layer F.Cu) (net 2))
 (segment (start 130.81 119.38) (end 130.81 120.6053) (width 0.25) (layer B.Cu) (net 2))
 (segment (start 157.48 118.1547) (end 166.37 118.1547) (width 0.25) (layer B.Cu) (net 2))
 (segment (start 157.48 119.38) (end 157.48 118.1547) (width 0.25) (layer B.Cu) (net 2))
 (segment (start 148.59 120.6053) (end 157.48 120.6053) (width 0.25) (layer B.Cu) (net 2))
 (segment (start 157.48 119.38) (end 157.48 120.6053) (width 0.25) (layer B.Cu) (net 2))
 (segment (start 126.3203 120.6053) (end 130.81 120.6053) (width 0.25) (layer B.Cu) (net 2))
 (segment (start 124.46 118.745) (end 126.3203 120.6053) (width 0.25) (layer B.Cu) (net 2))
 (segment (start 130.81 120.6053) (end 139.7 120.6053) (width 0.25) (layer B.Cu) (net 2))
 (segment (start 139.7 119.38) (end 139.7 120.6053) (width 0.25) (layer B.Cu) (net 2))
 (segment (start 148.59 119.38) (end 148.59 120.4927) (width 0.25) (layer B.Cu) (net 2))
 (segment (start 148.59 120.4927) (end 148.59 120.6053) (width 0.25) (layer B.Cu) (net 2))
 (segment (start 148.59 120.6053) (end 139.7 120.6053) (width 0.25) (layer B.Cu) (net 2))
 (segment (start 148.6695 106.0212) (end 151.8207 102.87) (width 0.25) (layer F.Cu) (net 2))
 (segment (start 148.6695 118.0752) (end 148.6695 106.0212) (width 0.25) (layer F.Cu) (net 2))
 (segment (start 148.59 118.1547) (end 148.6695 118.0752) (width 0.25) (layer F.Cu) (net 2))
 (segment (start 148.59 119.38) (end 148.59 118.1547) (width 0.25) (layer F.Cu) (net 2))
 (segment (start 166.37 119.38) (end 166.37 118.2673) (width 0.25) (layer B.Cu) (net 2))
 (segment (start 166.37 118.2673) (end 166.37 118.1547) (width 0.25) (layer B.Cu) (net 2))
 (segment (start 168.2193 108.651) (end 168.2193 102.87) (width 0.25) (layer B.Cu) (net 2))
 (segment (start 166.37 110.5003) (end 168.2193 108.651) (width 0.25) (layer B.Cu) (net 2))
 (segment (start 166.37 118.1547) (end 166.37 110.5003) (width 0.25) (layer B.Cu) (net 2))
 (segment (start 166.37 102.87) (end 168.2193 102.87) (width 0.25) (layer B.Cu) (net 2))
 (segment (start 132.08 107.95) (end 144.78 107.95) (width 0.25) (layer B.Cu) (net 22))
 (segment (start 136.9754 74.8754) (end 135.89 73.79) (width 0.25) (layer F.Cu) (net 22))
 (segment (start 136.9754 86.1982) (end 136.9754 74.8754) (width 0.25) (layer F.Cu) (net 22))
 (segment (start 133.6563 89.5173) (end 136.9754 86.1982) (width 0.25) (layer F.Cu) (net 22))
 (segment (start 133.6563 93.5392) (end 133.6563 89.5173) (width 0.25) (layer F.Cu) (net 22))
 (segment (start 133.9293 93.8122) (end 133.6563 93.5392) (width 0.25) (layer F.Cu) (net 22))
 (segment (start 133.9293 107.95) (end 133.9293 93.8122) (width 0.25) (layer F.Cu) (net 22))
 (segment (start 132.08 107.95) (end 133.9293 107.95) (width 0.25) (layer F.Cu) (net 22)))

